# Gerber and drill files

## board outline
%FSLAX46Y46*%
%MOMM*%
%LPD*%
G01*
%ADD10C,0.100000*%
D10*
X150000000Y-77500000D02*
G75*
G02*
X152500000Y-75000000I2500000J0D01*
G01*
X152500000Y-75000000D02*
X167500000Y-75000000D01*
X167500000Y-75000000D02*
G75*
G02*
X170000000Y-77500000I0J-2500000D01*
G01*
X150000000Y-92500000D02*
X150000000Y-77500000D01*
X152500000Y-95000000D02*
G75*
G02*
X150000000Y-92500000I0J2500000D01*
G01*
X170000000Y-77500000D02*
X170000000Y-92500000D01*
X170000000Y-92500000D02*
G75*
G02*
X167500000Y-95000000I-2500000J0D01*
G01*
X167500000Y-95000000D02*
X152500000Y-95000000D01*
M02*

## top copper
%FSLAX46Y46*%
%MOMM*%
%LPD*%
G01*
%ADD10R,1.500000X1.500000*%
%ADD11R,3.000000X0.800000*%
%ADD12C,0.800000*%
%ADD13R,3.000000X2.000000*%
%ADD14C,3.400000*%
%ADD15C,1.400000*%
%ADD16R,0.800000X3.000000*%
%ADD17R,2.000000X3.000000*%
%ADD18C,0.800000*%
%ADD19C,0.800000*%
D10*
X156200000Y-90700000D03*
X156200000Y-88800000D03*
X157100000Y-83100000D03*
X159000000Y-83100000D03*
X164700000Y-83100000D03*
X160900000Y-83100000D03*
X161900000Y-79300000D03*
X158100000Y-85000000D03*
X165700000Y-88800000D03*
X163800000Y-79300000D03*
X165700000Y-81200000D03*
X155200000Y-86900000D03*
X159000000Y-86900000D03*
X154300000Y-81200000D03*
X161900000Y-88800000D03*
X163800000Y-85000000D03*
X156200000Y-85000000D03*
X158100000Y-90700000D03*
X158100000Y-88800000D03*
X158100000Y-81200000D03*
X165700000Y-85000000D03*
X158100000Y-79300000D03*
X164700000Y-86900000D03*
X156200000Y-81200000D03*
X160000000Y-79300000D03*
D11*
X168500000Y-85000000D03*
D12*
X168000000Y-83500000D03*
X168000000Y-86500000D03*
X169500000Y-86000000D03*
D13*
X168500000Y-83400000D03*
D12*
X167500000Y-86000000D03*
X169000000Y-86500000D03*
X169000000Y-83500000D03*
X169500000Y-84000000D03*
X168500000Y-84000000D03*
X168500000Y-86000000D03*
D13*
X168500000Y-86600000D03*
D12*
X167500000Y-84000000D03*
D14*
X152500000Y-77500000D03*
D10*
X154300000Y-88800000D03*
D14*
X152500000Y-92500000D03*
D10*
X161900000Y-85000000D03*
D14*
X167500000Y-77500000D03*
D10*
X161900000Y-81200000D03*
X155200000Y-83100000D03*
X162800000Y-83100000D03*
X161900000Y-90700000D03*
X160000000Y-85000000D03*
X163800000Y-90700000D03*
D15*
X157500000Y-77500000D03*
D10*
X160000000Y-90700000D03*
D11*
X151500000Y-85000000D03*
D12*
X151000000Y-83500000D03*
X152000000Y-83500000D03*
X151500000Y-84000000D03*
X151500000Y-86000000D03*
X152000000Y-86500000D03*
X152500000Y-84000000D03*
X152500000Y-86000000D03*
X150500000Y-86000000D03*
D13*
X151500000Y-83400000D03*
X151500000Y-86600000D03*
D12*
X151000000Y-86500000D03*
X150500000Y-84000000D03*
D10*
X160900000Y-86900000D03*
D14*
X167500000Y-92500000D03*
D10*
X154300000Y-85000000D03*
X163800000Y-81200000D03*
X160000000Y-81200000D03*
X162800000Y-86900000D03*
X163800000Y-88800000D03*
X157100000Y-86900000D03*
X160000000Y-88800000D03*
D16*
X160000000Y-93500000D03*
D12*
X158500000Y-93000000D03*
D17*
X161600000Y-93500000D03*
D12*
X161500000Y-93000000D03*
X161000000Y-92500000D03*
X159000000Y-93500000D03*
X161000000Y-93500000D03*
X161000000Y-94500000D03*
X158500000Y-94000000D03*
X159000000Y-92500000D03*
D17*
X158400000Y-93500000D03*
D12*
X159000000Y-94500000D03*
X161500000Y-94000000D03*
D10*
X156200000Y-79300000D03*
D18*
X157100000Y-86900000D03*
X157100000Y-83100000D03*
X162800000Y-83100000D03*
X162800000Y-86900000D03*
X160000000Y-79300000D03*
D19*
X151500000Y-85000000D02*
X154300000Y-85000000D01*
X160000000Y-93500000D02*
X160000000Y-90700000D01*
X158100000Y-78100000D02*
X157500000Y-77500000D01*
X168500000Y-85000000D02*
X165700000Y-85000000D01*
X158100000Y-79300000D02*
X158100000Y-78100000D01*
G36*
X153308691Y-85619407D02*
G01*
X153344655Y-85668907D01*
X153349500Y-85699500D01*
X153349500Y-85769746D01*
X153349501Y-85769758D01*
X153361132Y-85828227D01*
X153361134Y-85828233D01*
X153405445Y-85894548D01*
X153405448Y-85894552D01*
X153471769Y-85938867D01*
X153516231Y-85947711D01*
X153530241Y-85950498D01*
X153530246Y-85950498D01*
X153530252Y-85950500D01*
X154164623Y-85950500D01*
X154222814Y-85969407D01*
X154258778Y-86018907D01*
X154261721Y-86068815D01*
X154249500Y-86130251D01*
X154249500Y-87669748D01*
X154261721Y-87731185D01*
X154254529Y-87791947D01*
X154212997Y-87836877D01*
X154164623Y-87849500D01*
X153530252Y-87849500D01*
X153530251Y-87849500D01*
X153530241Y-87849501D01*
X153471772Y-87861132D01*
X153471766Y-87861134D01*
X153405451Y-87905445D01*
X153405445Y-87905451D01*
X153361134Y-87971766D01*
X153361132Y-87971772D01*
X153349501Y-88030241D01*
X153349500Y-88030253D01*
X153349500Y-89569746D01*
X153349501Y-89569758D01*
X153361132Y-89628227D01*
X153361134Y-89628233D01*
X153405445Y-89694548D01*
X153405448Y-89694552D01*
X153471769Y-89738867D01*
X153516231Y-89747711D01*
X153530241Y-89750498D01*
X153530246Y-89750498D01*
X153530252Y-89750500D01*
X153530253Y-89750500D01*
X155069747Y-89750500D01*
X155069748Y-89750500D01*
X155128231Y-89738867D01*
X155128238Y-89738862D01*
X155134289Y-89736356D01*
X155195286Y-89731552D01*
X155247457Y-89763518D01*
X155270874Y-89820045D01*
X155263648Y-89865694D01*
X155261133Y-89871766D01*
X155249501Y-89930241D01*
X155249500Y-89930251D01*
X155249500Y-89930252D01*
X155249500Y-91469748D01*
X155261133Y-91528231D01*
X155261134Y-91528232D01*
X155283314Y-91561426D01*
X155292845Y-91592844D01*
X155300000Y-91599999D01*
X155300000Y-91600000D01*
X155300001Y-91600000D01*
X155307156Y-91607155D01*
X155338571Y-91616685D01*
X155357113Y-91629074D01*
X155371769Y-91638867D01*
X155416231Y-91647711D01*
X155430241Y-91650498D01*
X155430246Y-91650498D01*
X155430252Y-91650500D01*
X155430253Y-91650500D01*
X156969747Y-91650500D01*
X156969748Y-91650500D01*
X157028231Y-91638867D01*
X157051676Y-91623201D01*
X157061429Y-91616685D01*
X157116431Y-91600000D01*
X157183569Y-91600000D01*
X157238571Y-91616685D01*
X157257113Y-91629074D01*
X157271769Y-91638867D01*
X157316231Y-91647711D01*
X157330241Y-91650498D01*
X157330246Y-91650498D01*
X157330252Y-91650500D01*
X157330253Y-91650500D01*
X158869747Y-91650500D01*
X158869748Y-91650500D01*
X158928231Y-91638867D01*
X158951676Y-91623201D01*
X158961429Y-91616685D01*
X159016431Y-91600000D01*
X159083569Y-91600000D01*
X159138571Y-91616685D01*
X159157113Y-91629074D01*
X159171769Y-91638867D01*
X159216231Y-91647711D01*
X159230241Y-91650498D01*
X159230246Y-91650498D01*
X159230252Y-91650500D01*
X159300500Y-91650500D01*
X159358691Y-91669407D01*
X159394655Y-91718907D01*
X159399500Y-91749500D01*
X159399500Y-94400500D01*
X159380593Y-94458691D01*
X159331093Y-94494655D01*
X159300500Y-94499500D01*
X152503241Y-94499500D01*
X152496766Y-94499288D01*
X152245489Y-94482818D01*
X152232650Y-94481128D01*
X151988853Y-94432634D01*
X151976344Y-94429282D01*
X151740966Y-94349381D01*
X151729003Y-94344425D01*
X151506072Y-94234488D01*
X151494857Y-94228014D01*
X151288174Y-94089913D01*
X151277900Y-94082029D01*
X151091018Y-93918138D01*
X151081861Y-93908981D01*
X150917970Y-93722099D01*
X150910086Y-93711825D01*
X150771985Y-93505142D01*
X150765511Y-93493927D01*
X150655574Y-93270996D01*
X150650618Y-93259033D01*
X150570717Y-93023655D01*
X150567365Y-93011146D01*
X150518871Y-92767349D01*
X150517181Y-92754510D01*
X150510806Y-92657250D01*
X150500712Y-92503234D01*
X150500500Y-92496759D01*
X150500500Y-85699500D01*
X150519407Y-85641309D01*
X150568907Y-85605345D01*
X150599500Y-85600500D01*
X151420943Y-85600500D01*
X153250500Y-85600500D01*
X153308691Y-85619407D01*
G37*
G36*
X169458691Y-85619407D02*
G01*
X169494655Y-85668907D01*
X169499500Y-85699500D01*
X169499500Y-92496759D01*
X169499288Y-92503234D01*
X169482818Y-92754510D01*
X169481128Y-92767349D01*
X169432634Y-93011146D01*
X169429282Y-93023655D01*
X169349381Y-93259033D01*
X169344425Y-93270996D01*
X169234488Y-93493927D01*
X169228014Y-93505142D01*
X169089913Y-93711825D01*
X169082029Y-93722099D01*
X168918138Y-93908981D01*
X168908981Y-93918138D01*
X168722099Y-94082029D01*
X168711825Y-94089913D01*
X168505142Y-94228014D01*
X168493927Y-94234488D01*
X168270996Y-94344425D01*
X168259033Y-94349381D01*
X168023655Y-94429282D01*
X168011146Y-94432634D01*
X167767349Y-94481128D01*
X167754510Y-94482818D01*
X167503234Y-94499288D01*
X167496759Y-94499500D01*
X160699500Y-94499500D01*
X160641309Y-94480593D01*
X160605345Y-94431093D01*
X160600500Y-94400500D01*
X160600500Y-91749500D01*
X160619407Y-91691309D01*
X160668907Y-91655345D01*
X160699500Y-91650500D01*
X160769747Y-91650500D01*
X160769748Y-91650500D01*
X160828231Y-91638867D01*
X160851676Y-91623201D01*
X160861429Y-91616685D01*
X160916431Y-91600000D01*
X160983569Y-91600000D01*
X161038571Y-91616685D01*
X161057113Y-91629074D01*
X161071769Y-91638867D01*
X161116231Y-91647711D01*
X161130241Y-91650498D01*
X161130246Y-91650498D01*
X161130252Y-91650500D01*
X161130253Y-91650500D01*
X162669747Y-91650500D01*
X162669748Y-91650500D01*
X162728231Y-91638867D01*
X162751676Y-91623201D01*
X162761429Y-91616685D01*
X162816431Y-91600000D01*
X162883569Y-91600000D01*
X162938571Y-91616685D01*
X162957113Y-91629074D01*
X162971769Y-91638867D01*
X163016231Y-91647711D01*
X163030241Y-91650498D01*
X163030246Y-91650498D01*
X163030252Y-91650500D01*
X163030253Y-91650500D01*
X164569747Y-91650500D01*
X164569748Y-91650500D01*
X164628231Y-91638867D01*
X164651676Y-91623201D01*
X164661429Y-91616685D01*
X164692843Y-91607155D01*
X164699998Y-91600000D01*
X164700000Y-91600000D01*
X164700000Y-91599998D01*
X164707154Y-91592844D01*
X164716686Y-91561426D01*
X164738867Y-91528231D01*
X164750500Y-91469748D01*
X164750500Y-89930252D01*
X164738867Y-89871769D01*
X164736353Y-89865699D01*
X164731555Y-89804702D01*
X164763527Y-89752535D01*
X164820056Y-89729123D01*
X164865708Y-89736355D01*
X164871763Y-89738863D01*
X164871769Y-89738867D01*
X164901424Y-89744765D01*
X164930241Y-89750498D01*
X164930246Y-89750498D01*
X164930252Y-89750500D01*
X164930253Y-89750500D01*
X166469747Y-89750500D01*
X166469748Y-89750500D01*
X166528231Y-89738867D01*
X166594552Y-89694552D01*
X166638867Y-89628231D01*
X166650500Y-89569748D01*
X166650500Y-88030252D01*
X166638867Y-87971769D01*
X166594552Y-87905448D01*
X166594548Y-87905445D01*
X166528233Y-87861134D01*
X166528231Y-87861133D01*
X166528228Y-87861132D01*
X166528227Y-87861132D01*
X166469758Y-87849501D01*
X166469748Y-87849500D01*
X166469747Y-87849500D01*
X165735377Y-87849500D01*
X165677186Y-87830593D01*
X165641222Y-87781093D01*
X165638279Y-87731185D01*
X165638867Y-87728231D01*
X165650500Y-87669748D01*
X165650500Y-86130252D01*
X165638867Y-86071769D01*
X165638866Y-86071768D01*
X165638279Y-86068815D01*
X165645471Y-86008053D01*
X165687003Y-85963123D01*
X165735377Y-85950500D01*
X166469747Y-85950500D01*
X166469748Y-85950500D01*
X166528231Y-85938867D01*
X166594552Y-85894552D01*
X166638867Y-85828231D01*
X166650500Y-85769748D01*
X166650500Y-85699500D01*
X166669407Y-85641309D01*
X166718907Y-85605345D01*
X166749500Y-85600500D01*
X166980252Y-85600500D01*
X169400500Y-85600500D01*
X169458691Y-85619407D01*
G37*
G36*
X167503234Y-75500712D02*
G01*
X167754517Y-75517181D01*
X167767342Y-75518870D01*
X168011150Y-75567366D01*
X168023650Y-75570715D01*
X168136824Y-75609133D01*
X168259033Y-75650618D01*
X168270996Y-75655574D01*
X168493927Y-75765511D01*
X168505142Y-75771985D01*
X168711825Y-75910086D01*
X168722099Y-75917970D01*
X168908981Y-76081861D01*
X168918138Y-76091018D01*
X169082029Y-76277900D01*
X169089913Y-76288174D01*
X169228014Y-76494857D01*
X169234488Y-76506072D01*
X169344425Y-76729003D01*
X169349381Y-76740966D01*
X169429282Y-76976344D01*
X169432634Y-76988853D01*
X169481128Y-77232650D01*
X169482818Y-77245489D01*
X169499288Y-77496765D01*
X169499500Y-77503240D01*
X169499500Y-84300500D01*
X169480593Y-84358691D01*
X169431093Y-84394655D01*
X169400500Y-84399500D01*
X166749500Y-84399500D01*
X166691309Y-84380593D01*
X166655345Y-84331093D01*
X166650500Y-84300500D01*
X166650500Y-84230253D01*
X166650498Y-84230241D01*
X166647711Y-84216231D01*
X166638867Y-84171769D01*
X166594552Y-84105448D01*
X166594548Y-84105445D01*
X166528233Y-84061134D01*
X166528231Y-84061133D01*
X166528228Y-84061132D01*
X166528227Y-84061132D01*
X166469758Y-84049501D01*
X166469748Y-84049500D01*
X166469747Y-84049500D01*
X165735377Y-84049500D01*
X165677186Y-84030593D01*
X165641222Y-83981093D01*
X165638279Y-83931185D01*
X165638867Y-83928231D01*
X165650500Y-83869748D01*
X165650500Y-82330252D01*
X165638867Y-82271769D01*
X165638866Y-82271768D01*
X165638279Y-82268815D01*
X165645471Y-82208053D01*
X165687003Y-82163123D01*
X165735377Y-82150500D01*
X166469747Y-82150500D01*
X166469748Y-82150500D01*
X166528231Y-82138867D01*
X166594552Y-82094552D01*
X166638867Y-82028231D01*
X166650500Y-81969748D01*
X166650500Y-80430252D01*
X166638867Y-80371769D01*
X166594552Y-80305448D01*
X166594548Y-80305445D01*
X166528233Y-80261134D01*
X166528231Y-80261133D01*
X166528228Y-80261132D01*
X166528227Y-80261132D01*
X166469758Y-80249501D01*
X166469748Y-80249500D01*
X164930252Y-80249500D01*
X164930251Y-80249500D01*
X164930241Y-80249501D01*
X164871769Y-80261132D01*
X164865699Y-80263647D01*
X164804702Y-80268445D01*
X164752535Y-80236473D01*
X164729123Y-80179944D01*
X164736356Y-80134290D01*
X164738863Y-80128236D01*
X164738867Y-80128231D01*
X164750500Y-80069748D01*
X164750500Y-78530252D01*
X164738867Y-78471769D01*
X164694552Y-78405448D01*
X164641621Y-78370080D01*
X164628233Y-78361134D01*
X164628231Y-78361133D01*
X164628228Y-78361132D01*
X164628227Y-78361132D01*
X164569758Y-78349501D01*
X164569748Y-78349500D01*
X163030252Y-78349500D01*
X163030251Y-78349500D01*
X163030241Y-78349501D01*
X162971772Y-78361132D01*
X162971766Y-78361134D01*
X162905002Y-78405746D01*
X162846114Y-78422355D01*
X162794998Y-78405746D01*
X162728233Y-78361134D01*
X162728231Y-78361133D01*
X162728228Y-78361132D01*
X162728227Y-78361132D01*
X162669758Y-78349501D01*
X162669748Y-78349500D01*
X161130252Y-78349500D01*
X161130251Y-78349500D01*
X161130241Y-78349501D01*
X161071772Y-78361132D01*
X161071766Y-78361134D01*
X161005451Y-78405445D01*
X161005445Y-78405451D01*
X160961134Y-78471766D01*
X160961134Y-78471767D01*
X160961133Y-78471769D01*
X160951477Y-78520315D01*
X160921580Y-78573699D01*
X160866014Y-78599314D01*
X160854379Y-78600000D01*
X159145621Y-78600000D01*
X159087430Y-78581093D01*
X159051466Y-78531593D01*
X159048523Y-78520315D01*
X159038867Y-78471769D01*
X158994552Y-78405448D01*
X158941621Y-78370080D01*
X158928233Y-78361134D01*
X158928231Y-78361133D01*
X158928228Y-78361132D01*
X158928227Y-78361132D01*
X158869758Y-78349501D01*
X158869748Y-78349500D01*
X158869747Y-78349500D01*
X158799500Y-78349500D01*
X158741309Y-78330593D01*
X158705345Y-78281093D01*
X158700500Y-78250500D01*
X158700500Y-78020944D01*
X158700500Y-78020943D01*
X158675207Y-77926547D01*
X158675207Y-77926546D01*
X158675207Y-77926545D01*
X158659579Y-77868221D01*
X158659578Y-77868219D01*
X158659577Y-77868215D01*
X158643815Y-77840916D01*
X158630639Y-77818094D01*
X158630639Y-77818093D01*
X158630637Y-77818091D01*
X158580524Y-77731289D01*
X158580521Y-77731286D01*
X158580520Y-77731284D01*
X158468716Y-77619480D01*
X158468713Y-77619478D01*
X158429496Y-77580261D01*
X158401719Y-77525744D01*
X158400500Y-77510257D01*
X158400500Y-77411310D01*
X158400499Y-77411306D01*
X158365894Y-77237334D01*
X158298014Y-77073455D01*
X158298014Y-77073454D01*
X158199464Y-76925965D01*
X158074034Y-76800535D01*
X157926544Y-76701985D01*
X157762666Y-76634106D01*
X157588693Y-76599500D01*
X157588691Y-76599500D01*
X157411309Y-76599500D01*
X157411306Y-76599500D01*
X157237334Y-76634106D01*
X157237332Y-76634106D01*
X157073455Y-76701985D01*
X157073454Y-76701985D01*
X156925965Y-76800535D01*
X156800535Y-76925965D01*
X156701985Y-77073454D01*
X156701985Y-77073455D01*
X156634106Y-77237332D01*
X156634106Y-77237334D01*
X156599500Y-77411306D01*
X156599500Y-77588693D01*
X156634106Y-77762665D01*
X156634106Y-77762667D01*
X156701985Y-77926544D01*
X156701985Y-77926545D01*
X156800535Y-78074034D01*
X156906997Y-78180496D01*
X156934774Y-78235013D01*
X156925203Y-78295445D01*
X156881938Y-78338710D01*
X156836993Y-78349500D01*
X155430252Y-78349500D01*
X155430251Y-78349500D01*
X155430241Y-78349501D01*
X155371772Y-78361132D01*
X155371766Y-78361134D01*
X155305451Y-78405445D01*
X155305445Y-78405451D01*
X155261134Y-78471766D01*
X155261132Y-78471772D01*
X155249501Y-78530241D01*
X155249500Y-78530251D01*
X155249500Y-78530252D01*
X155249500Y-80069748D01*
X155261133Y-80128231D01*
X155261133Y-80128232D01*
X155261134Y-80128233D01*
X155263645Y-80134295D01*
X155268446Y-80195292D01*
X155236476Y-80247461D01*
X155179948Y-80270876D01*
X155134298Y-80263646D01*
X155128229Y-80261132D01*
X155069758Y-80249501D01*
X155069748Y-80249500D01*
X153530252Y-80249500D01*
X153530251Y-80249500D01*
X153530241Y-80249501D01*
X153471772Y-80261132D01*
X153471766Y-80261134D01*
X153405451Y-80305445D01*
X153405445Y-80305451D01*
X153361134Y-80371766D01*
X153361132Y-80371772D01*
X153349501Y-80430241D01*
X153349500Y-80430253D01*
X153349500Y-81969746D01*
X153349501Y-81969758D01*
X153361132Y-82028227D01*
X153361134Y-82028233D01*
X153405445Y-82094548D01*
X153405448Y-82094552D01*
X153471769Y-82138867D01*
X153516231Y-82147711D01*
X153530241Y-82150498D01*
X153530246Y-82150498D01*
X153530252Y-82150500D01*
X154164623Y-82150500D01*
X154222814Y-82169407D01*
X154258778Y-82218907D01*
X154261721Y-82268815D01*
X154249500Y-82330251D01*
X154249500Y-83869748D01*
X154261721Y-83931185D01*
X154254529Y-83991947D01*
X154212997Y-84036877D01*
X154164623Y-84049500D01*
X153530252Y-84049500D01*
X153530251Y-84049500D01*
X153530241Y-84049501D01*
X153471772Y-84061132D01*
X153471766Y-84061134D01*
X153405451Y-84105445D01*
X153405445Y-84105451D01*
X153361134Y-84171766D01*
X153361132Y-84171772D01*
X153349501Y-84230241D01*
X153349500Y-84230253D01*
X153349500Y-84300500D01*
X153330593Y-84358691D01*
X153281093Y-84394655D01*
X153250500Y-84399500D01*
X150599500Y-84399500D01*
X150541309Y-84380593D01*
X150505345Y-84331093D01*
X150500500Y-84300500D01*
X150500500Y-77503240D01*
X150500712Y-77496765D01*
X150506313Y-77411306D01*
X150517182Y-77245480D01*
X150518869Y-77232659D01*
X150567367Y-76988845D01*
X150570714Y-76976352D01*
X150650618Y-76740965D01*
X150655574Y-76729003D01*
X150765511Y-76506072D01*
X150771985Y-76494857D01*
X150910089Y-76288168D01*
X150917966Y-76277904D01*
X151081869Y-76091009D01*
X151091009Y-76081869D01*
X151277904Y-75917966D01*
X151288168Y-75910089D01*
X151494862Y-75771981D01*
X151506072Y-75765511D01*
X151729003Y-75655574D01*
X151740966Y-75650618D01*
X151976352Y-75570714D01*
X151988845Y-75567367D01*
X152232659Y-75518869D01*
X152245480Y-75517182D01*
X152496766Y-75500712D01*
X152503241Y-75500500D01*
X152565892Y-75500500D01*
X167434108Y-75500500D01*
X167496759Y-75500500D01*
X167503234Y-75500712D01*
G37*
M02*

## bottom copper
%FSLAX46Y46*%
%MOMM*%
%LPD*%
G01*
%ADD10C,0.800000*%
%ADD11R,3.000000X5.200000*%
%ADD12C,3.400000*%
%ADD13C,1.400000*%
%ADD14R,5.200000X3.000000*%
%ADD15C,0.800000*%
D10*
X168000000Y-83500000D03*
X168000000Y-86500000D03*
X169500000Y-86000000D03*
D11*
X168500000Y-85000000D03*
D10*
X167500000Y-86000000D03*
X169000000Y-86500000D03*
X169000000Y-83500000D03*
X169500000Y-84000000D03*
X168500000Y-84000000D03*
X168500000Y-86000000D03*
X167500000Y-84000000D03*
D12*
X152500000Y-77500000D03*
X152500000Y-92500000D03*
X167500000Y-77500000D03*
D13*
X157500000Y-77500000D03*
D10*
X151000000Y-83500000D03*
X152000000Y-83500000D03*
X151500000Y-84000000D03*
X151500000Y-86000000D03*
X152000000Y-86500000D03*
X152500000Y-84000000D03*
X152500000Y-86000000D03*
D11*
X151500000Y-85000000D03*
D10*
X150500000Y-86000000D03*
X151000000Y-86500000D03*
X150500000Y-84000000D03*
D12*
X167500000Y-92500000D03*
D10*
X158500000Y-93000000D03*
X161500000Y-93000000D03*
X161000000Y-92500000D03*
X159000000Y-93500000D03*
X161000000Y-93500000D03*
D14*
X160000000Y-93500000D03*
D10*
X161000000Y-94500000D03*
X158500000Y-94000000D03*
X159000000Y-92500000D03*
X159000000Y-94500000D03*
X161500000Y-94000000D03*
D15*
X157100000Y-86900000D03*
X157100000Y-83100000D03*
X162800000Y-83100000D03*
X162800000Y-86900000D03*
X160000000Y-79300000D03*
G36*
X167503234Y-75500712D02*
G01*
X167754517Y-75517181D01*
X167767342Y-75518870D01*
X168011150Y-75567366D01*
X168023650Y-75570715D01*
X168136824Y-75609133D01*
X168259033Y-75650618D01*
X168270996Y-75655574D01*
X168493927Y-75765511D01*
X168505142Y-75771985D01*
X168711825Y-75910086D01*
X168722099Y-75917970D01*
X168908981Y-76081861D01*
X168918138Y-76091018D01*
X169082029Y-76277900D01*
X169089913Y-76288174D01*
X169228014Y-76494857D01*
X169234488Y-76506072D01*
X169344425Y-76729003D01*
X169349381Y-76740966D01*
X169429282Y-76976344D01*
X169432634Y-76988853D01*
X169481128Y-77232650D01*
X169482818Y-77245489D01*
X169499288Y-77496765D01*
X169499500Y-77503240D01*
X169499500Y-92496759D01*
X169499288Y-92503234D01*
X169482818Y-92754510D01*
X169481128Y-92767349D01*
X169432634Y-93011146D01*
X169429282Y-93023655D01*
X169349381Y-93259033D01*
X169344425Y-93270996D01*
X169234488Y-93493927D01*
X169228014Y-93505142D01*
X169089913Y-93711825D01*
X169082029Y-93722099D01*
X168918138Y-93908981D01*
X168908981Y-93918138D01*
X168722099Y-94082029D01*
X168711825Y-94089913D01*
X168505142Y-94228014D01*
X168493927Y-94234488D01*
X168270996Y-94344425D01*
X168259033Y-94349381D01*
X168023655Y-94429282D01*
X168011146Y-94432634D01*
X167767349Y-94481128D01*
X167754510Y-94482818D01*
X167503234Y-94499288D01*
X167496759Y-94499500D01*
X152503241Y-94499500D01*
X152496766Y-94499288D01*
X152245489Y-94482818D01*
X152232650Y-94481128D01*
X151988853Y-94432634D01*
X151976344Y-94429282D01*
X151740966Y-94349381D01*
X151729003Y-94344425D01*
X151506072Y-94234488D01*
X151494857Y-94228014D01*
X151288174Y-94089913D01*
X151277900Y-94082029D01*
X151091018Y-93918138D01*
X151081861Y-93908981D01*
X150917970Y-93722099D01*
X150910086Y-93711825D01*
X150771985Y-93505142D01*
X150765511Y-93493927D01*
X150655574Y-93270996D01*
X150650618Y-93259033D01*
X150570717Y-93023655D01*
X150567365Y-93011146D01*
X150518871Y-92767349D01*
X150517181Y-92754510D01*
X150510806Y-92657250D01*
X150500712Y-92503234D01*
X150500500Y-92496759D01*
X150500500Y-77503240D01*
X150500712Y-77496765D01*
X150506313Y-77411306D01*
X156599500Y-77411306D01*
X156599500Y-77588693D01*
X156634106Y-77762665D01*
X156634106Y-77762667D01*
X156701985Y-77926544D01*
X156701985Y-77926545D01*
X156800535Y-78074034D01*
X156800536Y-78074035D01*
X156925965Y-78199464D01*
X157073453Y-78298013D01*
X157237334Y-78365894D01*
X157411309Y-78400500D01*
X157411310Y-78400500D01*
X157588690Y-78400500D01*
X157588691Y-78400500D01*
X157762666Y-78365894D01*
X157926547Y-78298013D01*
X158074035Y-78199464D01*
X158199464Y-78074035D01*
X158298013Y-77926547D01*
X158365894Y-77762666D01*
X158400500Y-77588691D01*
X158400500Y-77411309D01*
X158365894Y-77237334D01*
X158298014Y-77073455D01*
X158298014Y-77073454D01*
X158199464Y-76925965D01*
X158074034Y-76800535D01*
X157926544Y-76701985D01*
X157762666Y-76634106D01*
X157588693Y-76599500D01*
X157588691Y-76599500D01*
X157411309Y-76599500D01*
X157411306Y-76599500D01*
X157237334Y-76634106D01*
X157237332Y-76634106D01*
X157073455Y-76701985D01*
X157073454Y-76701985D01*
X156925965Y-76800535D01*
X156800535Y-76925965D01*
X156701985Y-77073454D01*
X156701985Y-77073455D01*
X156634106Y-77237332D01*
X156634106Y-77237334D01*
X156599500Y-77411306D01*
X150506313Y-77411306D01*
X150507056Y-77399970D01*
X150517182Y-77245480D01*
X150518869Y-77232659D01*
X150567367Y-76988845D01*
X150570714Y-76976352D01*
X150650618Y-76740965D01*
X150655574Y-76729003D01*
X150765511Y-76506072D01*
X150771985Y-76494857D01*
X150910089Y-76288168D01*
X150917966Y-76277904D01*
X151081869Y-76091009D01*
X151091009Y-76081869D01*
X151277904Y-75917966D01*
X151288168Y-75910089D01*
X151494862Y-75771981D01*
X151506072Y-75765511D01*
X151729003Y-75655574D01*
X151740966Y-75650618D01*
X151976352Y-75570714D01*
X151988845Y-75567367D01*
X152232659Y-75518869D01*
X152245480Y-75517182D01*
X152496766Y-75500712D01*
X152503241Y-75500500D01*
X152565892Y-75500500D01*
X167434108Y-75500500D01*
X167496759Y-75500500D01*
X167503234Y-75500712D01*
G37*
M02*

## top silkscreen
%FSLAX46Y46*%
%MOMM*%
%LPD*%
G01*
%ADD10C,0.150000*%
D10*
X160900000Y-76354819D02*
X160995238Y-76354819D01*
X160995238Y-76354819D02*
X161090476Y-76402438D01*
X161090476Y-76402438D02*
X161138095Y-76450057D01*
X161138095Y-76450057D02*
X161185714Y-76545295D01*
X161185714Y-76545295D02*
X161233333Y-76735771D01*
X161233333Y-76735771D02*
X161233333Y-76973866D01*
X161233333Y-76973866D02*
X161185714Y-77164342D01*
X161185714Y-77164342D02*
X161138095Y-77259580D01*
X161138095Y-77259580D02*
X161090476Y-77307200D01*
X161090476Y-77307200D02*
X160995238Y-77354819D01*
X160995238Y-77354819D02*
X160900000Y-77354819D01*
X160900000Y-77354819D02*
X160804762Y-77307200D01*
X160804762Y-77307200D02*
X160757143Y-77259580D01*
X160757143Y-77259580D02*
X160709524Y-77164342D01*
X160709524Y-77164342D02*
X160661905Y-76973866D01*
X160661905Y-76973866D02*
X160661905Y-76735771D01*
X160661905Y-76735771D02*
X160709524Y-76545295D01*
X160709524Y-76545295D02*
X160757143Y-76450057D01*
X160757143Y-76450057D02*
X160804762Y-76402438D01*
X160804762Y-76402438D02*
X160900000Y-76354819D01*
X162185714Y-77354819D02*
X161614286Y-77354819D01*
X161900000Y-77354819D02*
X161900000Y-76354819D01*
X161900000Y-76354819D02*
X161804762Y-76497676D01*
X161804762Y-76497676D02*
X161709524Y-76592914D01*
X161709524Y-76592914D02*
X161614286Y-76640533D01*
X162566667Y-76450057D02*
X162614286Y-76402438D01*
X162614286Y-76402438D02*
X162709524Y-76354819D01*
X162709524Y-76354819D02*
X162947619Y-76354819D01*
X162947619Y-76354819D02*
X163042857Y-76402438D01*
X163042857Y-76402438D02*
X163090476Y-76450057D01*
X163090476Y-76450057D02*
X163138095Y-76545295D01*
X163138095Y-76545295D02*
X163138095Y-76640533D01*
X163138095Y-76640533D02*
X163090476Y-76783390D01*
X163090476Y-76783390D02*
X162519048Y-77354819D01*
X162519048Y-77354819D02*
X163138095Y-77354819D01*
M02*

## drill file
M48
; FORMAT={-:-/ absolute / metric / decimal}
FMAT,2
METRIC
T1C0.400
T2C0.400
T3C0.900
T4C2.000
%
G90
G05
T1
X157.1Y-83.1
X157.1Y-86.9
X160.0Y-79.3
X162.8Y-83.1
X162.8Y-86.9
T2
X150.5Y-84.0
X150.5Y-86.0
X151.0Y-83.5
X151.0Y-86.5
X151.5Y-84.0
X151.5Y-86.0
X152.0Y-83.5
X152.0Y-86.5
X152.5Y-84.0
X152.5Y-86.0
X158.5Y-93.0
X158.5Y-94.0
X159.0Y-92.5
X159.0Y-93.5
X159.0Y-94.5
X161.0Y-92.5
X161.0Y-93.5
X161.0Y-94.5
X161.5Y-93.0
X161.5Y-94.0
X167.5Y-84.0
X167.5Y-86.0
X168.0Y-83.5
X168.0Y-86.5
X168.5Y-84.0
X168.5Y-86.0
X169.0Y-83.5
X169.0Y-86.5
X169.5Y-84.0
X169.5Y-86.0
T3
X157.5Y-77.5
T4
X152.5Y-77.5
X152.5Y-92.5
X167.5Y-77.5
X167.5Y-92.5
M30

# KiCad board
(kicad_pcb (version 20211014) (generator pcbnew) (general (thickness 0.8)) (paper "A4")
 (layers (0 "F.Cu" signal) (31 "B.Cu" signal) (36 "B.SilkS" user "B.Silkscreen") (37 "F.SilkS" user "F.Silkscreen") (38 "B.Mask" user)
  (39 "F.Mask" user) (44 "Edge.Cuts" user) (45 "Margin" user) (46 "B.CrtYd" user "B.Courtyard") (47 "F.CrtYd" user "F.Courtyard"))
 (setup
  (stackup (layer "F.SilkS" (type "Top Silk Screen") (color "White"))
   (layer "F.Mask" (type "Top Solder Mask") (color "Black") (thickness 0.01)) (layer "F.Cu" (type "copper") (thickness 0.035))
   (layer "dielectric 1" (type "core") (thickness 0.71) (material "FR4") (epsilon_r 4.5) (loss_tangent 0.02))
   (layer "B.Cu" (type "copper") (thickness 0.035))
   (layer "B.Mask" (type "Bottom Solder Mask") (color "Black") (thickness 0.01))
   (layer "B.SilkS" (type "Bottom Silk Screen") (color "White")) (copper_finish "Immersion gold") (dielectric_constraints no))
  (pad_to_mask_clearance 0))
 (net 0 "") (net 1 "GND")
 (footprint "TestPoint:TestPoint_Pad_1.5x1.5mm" (layer "F.Cu") (at 156.2 90.7)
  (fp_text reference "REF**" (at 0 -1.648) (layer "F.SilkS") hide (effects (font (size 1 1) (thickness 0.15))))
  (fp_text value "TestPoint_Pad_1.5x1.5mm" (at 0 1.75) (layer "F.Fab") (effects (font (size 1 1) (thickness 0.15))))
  (pad "1" smd rect (at 0 0) (size 1.5 1.5) (layers "F.Cu" "F.Mask")))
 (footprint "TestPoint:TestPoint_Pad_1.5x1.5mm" (layer "F.Cu") (at 156.2 88.8)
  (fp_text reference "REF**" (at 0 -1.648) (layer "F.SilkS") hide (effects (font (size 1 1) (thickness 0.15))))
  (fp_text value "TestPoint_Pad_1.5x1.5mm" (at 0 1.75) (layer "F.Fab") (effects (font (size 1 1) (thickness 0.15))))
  (pad "1" smd rect (at 0 0) (size 1.5 1.5) (layers "F.Cu" "F.Mask")))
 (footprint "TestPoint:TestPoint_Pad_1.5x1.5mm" (layer "F.Cu") (at 157.1 83.1)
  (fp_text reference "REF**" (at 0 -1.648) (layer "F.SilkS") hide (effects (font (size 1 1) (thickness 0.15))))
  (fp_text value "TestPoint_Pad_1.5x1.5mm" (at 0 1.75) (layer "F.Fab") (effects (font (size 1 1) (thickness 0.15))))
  (pad "1" smd rect (at 0 0) (size 1.5 1.5) (layers "F.Cu" "F.Paste" "F.Mask") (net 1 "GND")))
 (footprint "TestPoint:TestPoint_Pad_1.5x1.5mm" (layer "F.Cu") (at 159 83.1)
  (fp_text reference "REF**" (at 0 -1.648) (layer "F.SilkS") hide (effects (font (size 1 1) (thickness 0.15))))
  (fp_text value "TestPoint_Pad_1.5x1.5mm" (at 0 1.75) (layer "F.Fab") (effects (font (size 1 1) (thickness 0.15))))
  (pad "1" smd rect (at 0 0) (size 1.5 1.5) (layers "F.Cu" "F.Mask")))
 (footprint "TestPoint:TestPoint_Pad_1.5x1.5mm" (layer "F.Cu") (at 164.7 83.1)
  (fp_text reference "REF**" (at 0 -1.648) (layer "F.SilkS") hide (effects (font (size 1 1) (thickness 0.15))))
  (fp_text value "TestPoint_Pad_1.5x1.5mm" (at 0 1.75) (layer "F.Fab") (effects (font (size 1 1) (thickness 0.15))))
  (pad "1" smd rect (at 0 0) (size 1.5 1.5) (layers "F.Cu" "F.Mask")))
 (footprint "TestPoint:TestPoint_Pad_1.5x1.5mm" (layer "F.Cu") (at 160.9 83.1)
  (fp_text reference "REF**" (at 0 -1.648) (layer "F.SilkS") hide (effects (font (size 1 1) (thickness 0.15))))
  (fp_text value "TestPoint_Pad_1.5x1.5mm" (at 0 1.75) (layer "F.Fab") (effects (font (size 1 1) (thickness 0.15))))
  (pad "1" smd rect (at 0 0) (size 1.5 1.5) (layers "F.Cu" "F.Mask")))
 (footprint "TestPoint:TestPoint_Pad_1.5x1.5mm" (layer "F.Cu") (at 161.9 79.3)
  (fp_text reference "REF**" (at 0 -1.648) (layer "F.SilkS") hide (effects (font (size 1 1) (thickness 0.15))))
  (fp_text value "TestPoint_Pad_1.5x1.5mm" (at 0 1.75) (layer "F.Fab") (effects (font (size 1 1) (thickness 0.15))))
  (pad "1" smd rect (at 0 0) (size 1.5 1.5) (layers "F.Cu" "F.Mask")))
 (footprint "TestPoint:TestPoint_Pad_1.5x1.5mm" (layer "F.Cu") (at 158.1 85)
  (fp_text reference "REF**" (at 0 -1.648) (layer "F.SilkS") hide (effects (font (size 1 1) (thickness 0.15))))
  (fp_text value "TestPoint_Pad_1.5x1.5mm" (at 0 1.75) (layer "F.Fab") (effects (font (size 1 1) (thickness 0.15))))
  (pad "1" smd rect (at 0 0) (size 1.5 1.5) (layers "F.Cu" "F.Mask")))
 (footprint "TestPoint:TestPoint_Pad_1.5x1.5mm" (layer "F.Cu") (at 165.7 88.8)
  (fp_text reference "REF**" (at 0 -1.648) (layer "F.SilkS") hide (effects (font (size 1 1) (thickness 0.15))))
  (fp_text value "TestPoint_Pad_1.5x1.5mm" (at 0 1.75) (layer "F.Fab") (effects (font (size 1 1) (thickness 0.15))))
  (pad "1" smd rect (at 0 0) (size 1.5 1.5) (layers "F.Cu" "F.Mask")))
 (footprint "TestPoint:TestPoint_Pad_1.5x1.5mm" (layer "F.Cu") (at 163.8 79.3)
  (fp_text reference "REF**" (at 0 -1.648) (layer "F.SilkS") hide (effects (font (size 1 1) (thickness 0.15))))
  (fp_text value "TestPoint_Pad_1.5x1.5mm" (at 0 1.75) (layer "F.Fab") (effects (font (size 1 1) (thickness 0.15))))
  (pad "1" smd rect (at 0 0) (size 1.5 1.5) (layers "F.Cu" "F.Mask")))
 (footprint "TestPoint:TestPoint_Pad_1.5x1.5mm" (layer "F.Cu") (at 165.7 81.2)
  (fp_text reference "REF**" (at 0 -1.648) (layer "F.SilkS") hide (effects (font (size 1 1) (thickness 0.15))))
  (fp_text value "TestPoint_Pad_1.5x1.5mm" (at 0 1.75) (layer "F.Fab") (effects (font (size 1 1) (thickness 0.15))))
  (pad "1" smd rect (at 0 0) (size 1.5 1.5) (layers "F.Cu" "F.Mask")))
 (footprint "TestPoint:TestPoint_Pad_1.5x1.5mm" (layer "F.Cu") (at 155.2 86.9)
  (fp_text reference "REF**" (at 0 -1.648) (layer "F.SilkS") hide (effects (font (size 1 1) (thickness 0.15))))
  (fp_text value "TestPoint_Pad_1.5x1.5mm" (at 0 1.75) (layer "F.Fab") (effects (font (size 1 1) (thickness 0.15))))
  (pad "1" smd rect (at 0 0) (size 1.5 1.5) (layers "F.Cu" "F.Mask")))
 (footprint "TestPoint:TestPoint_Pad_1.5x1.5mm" (layer "F.Cu") (at 159 86.9)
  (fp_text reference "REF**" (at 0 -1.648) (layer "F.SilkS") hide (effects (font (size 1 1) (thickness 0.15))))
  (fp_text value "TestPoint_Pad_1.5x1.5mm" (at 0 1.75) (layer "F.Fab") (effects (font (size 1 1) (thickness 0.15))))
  (pad "1" smd rect (at 0 0) (size 1.5 1.5) (layers "F.Cu" "F.Mask")))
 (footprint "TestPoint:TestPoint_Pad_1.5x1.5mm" (layer "F.Cu") (at 154.3 81.2)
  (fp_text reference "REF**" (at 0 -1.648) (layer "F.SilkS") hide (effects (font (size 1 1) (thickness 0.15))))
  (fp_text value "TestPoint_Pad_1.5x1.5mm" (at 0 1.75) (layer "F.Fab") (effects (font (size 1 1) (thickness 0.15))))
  (pad "1" smd rect (at 0 0) (size 1.5 1.5) (layers "F.Cu" "F.Mask")))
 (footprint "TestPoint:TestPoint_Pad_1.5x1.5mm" (layer "F.Cu") (at 161.9 88.8)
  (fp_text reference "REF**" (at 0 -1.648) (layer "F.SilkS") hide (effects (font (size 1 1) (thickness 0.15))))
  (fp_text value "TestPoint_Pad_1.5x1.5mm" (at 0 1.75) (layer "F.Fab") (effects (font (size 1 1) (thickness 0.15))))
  (pad "1" smd rect (at 0 0) (size 1.5 1.5) (layers "F.Cu" "F.Mask")))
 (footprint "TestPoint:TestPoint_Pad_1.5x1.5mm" (layer "F.Cu") (at 163.8 85)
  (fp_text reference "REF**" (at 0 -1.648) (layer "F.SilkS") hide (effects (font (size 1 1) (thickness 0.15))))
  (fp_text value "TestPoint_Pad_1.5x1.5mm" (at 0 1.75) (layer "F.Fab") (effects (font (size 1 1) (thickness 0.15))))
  (pad "1" smd rect (at 0 0) (size 1.5 1.5) (layers "F.Cu" "F.Mask")))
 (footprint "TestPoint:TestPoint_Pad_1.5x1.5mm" (layer "F.Cu") (at 156.2 85)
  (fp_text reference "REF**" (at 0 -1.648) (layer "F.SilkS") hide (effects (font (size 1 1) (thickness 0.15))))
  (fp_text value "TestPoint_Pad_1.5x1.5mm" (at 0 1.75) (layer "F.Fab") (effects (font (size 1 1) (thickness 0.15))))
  (pad "1" smd rect (at 0 0) (size 1.5 1.5) (layers "F.Cu" "F.Mask")))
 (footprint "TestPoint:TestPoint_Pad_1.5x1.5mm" (layer "F.Cu") (at 158.1 90.7)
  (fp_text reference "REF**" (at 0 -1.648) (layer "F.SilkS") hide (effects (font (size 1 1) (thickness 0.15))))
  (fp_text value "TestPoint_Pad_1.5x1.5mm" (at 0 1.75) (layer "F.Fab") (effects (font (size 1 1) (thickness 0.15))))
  (pad "1" smd rect (at 0 0) (size 1.5 1.5) (layers "F.Cu" "F.Mask")))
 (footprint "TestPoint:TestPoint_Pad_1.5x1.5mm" (layer "F.Cu") (at 158.1 88.8)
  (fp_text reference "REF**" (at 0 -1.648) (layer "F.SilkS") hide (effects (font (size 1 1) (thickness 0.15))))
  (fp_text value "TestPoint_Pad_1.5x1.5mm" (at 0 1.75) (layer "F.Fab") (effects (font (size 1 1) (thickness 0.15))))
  (pad "1" smd rect (at 0 0) (size 1.5 1.5) (layers "F.Cu" "F.Mask")))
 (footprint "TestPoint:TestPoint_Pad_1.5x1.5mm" (layer "F.Cu") (at 158.1 81.2)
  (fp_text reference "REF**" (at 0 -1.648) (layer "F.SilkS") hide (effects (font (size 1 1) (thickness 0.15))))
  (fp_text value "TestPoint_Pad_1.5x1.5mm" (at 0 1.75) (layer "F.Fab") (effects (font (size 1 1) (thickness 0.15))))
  (pad "1" smd rect (at 0 0) (size 1.5 1.5) (layers "F.Cu" "F.Mask")))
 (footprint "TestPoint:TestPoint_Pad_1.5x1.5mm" (layer "F.Cu") (at 165.7 85)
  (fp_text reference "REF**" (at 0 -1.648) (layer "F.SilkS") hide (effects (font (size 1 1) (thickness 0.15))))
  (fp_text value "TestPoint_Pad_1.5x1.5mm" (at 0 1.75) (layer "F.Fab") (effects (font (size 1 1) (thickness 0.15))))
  (pad "1" smd rect (at 0 0) (size 1.5 1.5) (layers "F.Cu" "F.Mask")))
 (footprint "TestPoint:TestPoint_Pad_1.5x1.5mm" (layer "F.Cu") (at 158.1 79.3)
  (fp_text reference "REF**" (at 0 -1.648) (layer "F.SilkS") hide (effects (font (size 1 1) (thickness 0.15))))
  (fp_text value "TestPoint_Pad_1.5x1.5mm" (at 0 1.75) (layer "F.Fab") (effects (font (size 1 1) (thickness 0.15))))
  (pad "1" smd rect (at 0 0) (size 1.5 1.5) (layers "F.Cu" "F.Mask")))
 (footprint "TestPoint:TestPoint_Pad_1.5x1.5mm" (layer "F.Cu") (at 164.7 86.9)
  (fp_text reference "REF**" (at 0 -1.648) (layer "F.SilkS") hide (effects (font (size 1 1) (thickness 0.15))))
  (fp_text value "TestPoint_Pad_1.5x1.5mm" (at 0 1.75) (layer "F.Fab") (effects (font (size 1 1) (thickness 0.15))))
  (pad "1" smd rect (at 0 0) (size 1.5 1.5) (layers "F.Cu" "F.Mask")))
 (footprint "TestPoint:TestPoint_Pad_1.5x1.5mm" (layer "F.Cu") (at 156.2 81.2)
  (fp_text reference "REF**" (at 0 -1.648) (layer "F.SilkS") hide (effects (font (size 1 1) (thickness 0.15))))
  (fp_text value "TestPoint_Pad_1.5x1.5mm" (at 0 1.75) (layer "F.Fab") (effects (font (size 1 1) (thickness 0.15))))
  (pad "1" smd rect (at 0 0) (size 1.5 1.5) (layers "F.Cu" "F.Mask")))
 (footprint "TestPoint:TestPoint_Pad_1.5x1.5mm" (layer "F.Cu") (at 160 79.3)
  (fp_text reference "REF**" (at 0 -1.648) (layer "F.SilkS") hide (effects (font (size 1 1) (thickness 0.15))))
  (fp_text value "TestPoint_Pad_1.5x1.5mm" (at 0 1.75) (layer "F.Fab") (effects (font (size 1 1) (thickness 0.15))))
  (pad "1" smd rect (at 0 0) (size 1.5 1.5) (layers "F.Cu" "F.Paste" "F.Mask") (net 1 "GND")))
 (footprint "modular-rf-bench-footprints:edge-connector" (layer "F.Cu") (at 170 85)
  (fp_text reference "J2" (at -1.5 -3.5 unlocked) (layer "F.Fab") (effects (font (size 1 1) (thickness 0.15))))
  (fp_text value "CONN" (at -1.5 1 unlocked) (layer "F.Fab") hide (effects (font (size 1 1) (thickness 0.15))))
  (pad "1" smd rect (at -1.5 0) (size 3 0.8) (layers "F.Cu"))
  (pad "2" thru_hole circle (at -2 -1.5) (size 0.8 0.8) (drill 0.4) (layers *.Cu) (remove_unused_layers) (keep_end_layers) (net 1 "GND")
   (zone_connect 2))
  (pad "2" thru_hole circle (at -2 1.5) (size 0.8 0.8) (drill 0.4) (layers *.Cu) (remove_unused_layers) (keep_end_layers) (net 1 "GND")
   (zone_connect 2))
  (pad "2" thru_hole circle (at -0.5 1) (size 0.8 0.8) (drill 0.4) (layers *.Cu) (remove_unused_layers) (keep_end_layers) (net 1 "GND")
   (zone_connect 2))
  (pad "2" smd rect (at -1.5 -1.6) (size 3 2) (layers "F.Cu") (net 1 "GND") (zone_connect 2))
  (pad "2" smd rect (at -1.5 0) (size 3 5.2) (layers "B.Cu") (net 1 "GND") (zone_connect 2))
  (pad "2" thru_hole circle (at -2.5 1) (size 0.8 0.8) (drill 0.4) (layers *.Cu) (remove_unused_layers) (keep_end_layers) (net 1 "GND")
   (zone_connect 2))
  (pad "2" thru_hole circle (at -1 1.5) (size 0.8 0.8) (drill 0.4) (layers *.Cu) (remove_unused_layers) (keep_end_layers) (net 1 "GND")
   (zone_connect 2))
  (pad "2" thru_hole circle (at -1 -1.5) (size 0.8 0.8) (drill 0.4) (layers *.Cu) (remove_unused_layers) (keep_end_layers) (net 1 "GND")
   (zone_connect 2))
  (pad "2" thru_hole circle (at -0.5 -1) (size 0.8 0.8) (drill 0.4) (layers *.Cu) (remove_unused_layers) (keep_end_layers) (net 1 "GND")
   (zone_connect 2))
  (pad "2" thru_hole circle (at -1.5 -1) (size 0.8 0.8) (drill 0.4) (layers *.Cu) (remove_unused_layers) (keep_end_layers) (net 1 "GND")
   (zone_connect 2))
  (pad "2" thru_hole circle (at -1.5 1) (size 0.8 0.8) (drill 0.4) (layers *.Cu) (remove_unused_layers) (keep_end_layers) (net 1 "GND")
   (zone_connect 2))
  (pad "2" smd rect (at -1.5 1.6) (size 3 2) (layers "F.Cu") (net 1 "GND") (zone_connect 2))
  (pad "2" thru_hole circle (at -2.5 -1) (size 0.8 0.8) (drill 0.4) (layers *.Cu) (remove_unused_layers) (keep_end_layers) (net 1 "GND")
   (zone_connect 2)))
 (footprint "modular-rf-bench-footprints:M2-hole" (layer "F.Cu") (at 152.5 77.5)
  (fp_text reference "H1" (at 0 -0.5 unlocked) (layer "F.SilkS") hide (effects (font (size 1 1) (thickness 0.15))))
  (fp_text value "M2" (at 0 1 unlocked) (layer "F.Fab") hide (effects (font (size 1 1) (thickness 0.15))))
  (pad "1" thru_hole circle (at 0 0) (size 3.4 3.4) (drill 2) (layers *.Cu *.Mask) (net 1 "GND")))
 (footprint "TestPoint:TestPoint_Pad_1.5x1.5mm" (layer "F.Cu") (at 154.3 88.8)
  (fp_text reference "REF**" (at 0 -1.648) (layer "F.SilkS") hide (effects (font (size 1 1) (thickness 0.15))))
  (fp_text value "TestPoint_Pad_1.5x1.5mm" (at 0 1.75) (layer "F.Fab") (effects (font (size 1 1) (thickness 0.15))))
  (pad "1" smd rect (at 0 0) (size 1.5 1.5) (layers "F.Cu" "F.Mask")))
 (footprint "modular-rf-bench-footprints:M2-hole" (layer "F.Cu") (at 152.5 92.5)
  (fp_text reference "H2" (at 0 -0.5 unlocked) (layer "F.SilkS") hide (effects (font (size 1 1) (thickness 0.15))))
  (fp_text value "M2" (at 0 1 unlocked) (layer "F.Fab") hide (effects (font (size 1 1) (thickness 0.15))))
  (pad "1" thru_hole circle (at 0 0) (size 3.4 3.4) (drill 2) (layers *.Cu *.Mask) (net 1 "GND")))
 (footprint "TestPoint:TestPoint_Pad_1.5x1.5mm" (layer "F.Cu") (at 161.9 85)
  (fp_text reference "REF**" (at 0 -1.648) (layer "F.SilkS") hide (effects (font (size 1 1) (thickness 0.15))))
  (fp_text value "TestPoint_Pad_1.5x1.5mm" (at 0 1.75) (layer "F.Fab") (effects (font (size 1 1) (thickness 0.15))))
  (pad "1" smd rect (at 0 0) (size 1.5 1.5) (layers "F.Cu" "F.Mask")))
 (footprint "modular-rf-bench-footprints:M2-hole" (layer "F.Cu") (at 167.5 77.5)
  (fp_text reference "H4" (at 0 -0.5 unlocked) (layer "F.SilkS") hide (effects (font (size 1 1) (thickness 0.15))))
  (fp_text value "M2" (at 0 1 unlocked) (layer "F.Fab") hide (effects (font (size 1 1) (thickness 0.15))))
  (pad "1" thru_hole circle (at 0 0) (size 3.4 3.4) (drill 2) (layers *.Cu *.Mask) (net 1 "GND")))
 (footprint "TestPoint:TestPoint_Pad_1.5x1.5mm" (layer "F.Cu") (at 161.9 81.2)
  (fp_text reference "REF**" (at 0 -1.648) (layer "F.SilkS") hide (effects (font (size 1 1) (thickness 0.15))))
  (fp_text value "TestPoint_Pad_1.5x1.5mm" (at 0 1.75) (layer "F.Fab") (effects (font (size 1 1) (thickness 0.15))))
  (pad "1" smd rect (at 0 0) (size 1.5 1.5) (layers "F.Cu" "F.Mask")))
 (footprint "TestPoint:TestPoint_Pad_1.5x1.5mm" (layer "F.Cu") (at 155.2 83.1)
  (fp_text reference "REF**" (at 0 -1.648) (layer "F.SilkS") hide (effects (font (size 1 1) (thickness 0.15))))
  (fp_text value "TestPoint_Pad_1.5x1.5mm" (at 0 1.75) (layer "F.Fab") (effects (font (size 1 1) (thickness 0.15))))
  (pad "1" smd rect (at 0 0) (size 1.5 1.5) (layers "F.Cu" "F.Mask")))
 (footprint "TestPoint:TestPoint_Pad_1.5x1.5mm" (layer "F.Cu") (at 162.8 83.1)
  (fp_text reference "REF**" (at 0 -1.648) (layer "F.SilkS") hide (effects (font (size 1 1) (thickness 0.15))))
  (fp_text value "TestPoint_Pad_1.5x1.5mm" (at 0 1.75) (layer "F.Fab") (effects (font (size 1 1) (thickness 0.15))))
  (pad "1" smd rect (at 0 0) (size 1.5 1.5) (layers "F.Cu" "F.Paste" "F.Mask") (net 1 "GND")))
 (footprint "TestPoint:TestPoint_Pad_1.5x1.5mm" (layer "F.Cu") (at 161.9 90.7)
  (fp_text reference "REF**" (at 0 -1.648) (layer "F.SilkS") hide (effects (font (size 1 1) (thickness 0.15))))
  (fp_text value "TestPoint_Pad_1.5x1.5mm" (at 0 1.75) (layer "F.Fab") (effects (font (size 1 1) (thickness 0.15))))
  (pad "1" smd rect (at 0 0) (size 1.5 1.5) (layers "F.Cu" "F.Mask")))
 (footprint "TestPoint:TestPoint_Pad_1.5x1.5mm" (layer "F.Cu") (at 160 85)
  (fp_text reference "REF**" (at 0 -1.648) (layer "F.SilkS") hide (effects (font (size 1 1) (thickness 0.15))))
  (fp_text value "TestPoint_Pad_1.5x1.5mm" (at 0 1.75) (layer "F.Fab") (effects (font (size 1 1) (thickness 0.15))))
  (pad "1" smd rect (at 0 0) (size 1.5 1.5) (layers "F.Cu" "F.Mask")))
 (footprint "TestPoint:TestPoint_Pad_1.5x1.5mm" (layer "F.Cu") (at 163.8 90.7)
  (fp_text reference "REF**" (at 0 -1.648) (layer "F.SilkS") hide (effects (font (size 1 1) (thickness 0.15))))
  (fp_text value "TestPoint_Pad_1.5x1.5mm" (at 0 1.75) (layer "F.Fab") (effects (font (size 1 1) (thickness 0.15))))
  (pad "1" smd rect (at 0 0) (size 1.5 1.5) (layers "F.Cu" "F.Mask")))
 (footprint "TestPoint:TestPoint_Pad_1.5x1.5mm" (layer "F.Cu") (at 157.5 77.5)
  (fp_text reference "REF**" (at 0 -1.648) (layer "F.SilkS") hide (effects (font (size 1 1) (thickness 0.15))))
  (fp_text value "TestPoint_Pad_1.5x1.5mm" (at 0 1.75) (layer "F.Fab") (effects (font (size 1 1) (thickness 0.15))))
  (pad "1" thru_hole circle (at 0 0) (size 1.4 1.4) (drill 0.9) (layers *.Cu *.Mask)))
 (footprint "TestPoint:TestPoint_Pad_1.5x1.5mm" (layer "F.Cu") (at 160 90.7)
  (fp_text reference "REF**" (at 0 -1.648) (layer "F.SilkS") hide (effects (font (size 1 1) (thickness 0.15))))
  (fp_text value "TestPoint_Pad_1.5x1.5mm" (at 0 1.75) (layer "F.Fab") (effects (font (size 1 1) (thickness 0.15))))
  (pad "1" smd rect (at 0 0) (size 1.5 1.5) (layers "F.Cu" "F.Mask")))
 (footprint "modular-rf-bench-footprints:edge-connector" (layer "F.Cu") (at 150 85 180)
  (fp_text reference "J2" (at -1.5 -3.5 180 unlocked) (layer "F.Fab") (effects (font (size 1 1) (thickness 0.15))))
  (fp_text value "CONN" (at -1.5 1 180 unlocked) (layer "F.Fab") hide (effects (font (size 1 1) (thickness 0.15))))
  (pad "1" smd rect (at -1.5 0 180) (size 3 0.8) (layers "F.Cu"))
  (pad "2" thru_hole circle (at -1 1.5 180) (size 0.8 0.8) (drill 0.4) (layers *.Cu) (remove_unused_layers) (keep_end_layers) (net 1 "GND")
   (zone_connect 2))
  (pad "2" thru_hole circle (at -2 1.5 180) (size 0.8 0.8) (drill 0.4) (layers *.Cu) (remove_unused_layers) (keep_end_layers) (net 1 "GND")
   (zone_connect 2))
  (pad "2" thru_hole circle (at -1.5 1 180) (size 0.8 0.8) (drill 0.4) (layers *.Cu) (remove_unused_layers) (keep_end_layers) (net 1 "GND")
   (zone_connect 2))
  (pad "2" thru_hole circle (at -1.5 -1 180) (size 0.8 0.8) (drill 0.4) (layers *.Cu) (remove_unused_layers) (keep_end_layers) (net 1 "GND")
   (zone_connect 2))
  (pad "2" thru_hole circle (at -2 -1.5 180) (size 0.8 0.8) (drill 0.4) (layers *.Cu) (remove_unused_layers) (keep_end_layers) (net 1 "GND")
   (zone_connect 2))
  (pad "2" thru_hole circle (at -2.5 1 180) (size 0.8 0.8) (drill 0.4) (layers *.Cu) (remove_unused_layers) (keep_end_layers) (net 1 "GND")
   (zone_connect 2))
  (pad "2" thru_hole circle (at -2.5 -1 180) (size 0.8 0.8) (drill 0.4) (layers *.Cu) (remove_unused_layers) (keep_end_layers) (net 1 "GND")
   (zone_connect 2))
  (pad "2" smd rect (at -1.5 0 180) (size 3 5.2) (layers "B.Cu") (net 1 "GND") (zone_connect 2))
  (pad "2" thru_hole circle (at -0.5 -1 180) (size 0.8 0.8) (drill 0.4) (layers *.Cu) (remove_unused_layers) (keep_end_layers) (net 1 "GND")
   (zone_connect 2))
  (pad "2" smd rect (at -1.5 1.6 180) (size 3 2) (layers "F.Cu") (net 1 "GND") (zone_connect 2))
  (pad "2" smd rect (at -1.5 -1.6 180) (size 3 2) (layers "F.Cu") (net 1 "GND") (zone_connect 2))
  (pad "2" thru_hole circle (at -1 -1.5 180) (size 0.8 0.8) (drill 0.4) (layers *.Cu) (remove_unused_layers) (keep_end_layers) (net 1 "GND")
   (zone_connect 2))
  (pad "2" thru_hole circle (at -0.5 1 180) (size 0.8 0.8) (drill 0.4) (layers *.Cu) (remove_unused_layers) (keep_end_layers) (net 1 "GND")
   (zone_connect 2)))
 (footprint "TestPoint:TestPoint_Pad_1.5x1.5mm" (layer "F.Cu") (at 160.9 86.9)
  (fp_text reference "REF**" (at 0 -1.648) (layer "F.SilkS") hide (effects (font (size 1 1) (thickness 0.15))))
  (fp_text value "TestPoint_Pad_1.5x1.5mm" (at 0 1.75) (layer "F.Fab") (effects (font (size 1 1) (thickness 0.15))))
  (pad "1" smd rect (at 0 0) (size 1.5 1.5) (layers "F.Cu" "F.Mask")))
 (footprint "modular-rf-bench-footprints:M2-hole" (layer "F.Cu") (at 167.5 92.5)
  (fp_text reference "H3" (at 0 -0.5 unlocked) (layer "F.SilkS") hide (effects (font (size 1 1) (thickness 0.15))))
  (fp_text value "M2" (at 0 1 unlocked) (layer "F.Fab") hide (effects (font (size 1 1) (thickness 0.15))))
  (pad "1" thru_hole circle (at 0 0) (size 3.4 3.4) (drill 2) (layers *.Cu *.Mask) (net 1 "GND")))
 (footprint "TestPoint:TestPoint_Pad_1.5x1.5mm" (layer "F.Cu") (at 154.3 85)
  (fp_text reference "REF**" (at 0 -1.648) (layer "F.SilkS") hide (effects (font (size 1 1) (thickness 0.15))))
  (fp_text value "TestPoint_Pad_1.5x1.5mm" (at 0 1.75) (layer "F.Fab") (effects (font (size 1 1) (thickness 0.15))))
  (pad "1" smd rect (at 0 0) (size 1.5 1.5) (layers "F.Cu" "F.Mask")))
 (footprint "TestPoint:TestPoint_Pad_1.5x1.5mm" (layer "F.Cu") (at 163.8 81.2)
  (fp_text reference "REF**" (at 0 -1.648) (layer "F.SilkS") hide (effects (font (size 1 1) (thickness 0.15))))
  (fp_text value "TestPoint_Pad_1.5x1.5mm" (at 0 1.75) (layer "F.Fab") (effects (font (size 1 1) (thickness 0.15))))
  (pad "1" smd rect (at 0 0) (size 1.5 1.5) (layers "F.Cu" "F.Mask")))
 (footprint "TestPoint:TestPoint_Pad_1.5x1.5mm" (layer "F.Cu") (at 160 81.2)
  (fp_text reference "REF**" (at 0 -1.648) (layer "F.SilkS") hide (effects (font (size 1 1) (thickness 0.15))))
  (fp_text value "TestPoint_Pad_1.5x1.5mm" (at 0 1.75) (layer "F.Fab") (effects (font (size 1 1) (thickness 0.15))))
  (pad "1" smd rect (at 0 0) (size 1.5 1.5) (layers "F.Cu" "F.Mask")))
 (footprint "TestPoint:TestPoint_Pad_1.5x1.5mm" (layer "F.Cu") (at 162.8 86.9)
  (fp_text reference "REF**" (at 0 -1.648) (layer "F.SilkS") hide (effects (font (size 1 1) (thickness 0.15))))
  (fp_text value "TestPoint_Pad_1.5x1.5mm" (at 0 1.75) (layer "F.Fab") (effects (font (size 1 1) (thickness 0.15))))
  (pad "1" smd rect (at 0 0) (size 1.5 1.5) (layers "F.Cu" "F.Paste" "F.Mask") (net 1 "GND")))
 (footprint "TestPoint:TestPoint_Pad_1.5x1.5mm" (layer "F.Cu") (at 163.8 88.8)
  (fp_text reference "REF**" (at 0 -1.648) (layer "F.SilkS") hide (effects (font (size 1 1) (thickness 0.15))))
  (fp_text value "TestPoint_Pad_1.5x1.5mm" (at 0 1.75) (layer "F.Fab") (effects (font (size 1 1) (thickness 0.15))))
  (pad "1" smd rect (at 0 0) (size 1.5 1.5) (layers "F.Cu" "F.Mask")))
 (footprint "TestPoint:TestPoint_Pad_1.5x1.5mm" (layer "F.Cu") (at 157.1 86.9)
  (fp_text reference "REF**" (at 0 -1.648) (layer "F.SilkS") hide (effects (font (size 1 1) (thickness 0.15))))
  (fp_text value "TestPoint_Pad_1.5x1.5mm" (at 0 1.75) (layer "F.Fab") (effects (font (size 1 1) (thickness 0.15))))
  (pad "1" smd rect (at 0 0) (size 1.5 1.5) (layers "F.Cu" "F.Paste" "F.Mask") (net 1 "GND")))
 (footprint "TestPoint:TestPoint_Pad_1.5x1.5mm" (layer "F.Cu") (at 160 88.8)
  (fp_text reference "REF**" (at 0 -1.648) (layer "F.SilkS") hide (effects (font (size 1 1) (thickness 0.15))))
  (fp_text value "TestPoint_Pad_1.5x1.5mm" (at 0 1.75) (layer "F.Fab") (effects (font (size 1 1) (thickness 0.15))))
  (pad "1" smd rect (at 0 0) (size 1.5 1.5) (layers "F.Cu" "F.Mask")))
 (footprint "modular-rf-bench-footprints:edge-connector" (layer "F.Cu") (at 160 95 -90)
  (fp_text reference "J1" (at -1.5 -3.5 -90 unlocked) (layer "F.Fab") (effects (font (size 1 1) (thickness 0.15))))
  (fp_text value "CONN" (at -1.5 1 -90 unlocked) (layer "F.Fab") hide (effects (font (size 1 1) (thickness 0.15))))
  (pad "1" smd rect (at -1.5 0 270) (size 3 0.8) (layers "F.Cu"))
  (pad "2" thru_hole circle (at -2 1.5 270) (size 0.8 0.8) (drill 0.4) (layers *.Cu) (remove_unused_layers) (keep_end_layers) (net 1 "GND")
   (zone_connect 2))
  (pad "2" smd rect (at -1.5 -1.6 270) (size 3 2) (layers "F.Cu") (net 1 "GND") (zone_connect 2))
  (pad "2" thru_hole circle (at -2 -1.5 270) (size 0.8 0.8) (drill 0.4) (layers *.Cu) (remove_unused_layers) (keep_end_layers) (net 1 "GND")
   (zone_connect 2))
  (pad "2" thru_hole circle (at -2.5 -1 270) (size 0.8 0.8) (drill 0.4) (layers *.Cu) (remove_unused_layers) (keep_end_layers) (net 1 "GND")
   (zone_connect 2))
  (pad "2" thru_hole circle (at -1.5 1 270) (size 0.8 0.8) (drill 0.4) (layers *.Cu) (remove_unused_layers) (keep_end_layers) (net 1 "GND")
   (zone_connect 2))
  (pad "2" thru_hole circle (at -1.5 -1 270) (size 0.8 0.8) (drill 0.4) (layers *.Cu) (remove_unused_layers) (keep_end_layers) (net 1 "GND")
   (zone_connect 2))
  (pad "2" smd rect (at -1.5 0 270) (size 3 5.2) (layers "B.Cu") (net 1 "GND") (zone_connect 2))
  (pad "2" thru_hole circle (at -0.5 -1 270) (size 0.8 0.8) (drill 0.4) (layers *.Cu) (remove_unused_layers) (keep_end_layers) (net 1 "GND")
   (zone_connect 2))
  (pad "2" thru_hole circle (at -1 1.5 270) (size 0.8 0.8) (drill 0.4) (layers *.Cu) (remove_unused_layers) (keep_end_layers) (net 1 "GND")
   (zone_connect 2))
  (pad "2" thru_hole circle (at -2.5 1 270) (size 0.8 0.8) (drill 0.4) (layers *.Cu) (remove_unused_layers) (keep_end_layers) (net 1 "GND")
   (zone_connect 2))
  (pad "2" smd rect (at -1.5 1.6 270) (size 3 2) (layers "F.Cu") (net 1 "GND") (zone_connect 2))
  (pad "2" thru_hole circle (at -0.5 1 270) (size 0.8 0.8) (drill 0.4) (layers *.Cu) (remove_unused_layers) (keep_end_layers) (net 1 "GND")
   (zone_connect 2))
  (pad "2" thru_hole circle (at -1 -1.5 270) (size 0.8 0.8) (drill 0.4) (layers *.Cu) (remove_unused_layers) (keep_end_layers) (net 1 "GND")
   (zone_connect 2)))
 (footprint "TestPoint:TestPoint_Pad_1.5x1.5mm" (layer "F.Cu") (at 156.2 79.3)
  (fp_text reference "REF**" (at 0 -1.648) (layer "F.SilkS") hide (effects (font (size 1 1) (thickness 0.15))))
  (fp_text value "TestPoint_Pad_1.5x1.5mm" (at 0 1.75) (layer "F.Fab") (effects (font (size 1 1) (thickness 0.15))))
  (pad "1" smd rect (at 0 0) (size 1.5 1.5) (layers "F.Cu" "F.Mask")))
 (gr_arc (start 150 77.5) (mid 150.732233 75.732233) (end 152.5 75) (layer "Edge.Cuts") (width 0.1))
 (gr_line (start 152.5 75) (end 167.5 75) (layer "Edge.Cuts") (width 0.1))
 (gr_arc (start 167.5 75) (mid 169.267767 75.732233) (end 170 77.5) (layer "Edge.Cuts") (width 0.1))
 (gr_line (start 150 92.5) (end 150 77.5) (layer "Edge.Cuts") (width 0.1))
 (gr_arc (start 152.5 95) (mid 150.732233 94.267767) (end 150 92.5) (layer "Edge.Cuts") (width 0.1))
 (gr_line (start 170 77.5) (end 170 92.5) (layer "Edge.Cuts") (width 0.1))
 (gr_arc (start 170 92.5) (mid 169.267767 94.267767) (end 167.5 95) (layer "Edge.Cuts") (width 0.1))
 (gr_line (start 167.5 95) (end 152.5 95) (layer "Edge.Cuts") (width 0.1))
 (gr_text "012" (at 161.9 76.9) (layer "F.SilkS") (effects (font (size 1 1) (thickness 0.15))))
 (segment (start 151.5 85) (end 154.3 85) (width 0.8) (layer "F.Cu") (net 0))
 (segment (start 160 93.5) (end 160 90.7) (width 0.8) (layer "F.Cu") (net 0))
 (segment (start 158.1 78.1) (end 157.5 77.5) (width 0.8) (layer "F.Cu") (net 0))
 (segment (start 168.5 85) (end 165.7 85) (width 0.8) (layer "F.Cu") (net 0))
 (segment (start 158.1 79.3) (end 158.1 78.1) (width 0.8) (layer "F.Cu") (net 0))
 (via (at 157.1 86.9) (size 0.8) (drill 0.4) (layers "F.Cu" "B.Cu") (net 1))
 (via (at 157.1 83.1) (size 0.8) (drill 0.4) (layers "F.Cu" "B.Cu") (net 1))
 (via (at 162.8 83.1) (size 0.8) (drill 0.4) (layers "F.Cu" "B.Cu") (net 1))
 (via (at 162.8 86.9) (size 0.8) (drill 0.4) (layers "F.Cu" "B.Cu") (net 1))
 (via (at 160 79.3) (size 0.8) (drill 0.4) (layers "F.Cu" "B.Cu") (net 1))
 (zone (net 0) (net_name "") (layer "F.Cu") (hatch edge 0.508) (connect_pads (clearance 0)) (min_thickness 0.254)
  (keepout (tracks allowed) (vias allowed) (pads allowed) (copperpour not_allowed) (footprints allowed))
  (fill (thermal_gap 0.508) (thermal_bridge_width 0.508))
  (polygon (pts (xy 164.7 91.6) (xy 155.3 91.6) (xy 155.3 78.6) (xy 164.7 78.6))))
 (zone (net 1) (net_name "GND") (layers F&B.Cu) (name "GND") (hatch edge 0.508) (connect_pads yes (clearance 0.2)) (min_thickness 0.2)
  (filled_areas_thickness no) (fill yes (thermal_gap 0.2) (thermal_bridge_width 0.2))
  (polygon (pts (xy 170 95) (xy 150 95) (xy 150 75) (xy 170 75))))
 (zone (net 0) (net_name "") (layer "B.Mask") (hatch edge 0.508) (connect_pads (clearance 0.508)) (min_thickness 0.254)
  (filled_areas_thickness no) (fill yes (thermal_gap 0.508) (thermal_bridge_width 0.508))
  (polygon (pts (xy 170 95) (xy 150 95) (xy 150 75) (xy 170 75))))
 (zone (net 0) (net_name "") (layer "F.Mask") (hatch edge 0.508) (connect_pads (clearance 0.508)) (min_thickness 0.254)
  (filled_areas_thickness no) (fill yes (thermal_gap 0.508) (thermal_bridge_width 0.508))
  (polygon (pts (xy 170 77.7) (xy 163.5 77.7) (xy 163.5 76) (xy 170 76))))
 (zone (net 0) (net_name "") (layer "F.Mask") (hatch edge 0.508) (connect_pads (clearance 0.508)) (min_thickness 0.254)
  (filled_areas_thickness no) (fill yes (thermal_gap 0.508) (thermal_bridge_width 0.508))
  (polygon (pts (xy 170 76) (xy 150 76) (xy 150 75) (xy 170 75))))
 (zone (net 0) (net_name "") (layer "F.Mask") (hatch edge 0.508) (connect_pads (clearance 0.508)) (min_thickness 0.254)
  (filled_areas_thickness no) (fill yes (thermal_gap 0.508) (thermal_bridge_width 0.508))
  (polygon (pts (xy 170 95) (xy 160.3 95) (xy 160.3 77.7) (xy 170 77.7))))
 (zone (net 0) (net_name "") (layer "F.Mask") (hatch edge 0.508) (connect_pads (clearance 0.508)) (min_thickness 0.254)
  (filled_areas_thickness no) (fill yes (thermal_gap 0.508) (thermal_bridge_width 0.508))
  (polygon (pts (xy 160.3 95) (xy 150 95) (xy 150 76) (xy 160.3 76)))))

